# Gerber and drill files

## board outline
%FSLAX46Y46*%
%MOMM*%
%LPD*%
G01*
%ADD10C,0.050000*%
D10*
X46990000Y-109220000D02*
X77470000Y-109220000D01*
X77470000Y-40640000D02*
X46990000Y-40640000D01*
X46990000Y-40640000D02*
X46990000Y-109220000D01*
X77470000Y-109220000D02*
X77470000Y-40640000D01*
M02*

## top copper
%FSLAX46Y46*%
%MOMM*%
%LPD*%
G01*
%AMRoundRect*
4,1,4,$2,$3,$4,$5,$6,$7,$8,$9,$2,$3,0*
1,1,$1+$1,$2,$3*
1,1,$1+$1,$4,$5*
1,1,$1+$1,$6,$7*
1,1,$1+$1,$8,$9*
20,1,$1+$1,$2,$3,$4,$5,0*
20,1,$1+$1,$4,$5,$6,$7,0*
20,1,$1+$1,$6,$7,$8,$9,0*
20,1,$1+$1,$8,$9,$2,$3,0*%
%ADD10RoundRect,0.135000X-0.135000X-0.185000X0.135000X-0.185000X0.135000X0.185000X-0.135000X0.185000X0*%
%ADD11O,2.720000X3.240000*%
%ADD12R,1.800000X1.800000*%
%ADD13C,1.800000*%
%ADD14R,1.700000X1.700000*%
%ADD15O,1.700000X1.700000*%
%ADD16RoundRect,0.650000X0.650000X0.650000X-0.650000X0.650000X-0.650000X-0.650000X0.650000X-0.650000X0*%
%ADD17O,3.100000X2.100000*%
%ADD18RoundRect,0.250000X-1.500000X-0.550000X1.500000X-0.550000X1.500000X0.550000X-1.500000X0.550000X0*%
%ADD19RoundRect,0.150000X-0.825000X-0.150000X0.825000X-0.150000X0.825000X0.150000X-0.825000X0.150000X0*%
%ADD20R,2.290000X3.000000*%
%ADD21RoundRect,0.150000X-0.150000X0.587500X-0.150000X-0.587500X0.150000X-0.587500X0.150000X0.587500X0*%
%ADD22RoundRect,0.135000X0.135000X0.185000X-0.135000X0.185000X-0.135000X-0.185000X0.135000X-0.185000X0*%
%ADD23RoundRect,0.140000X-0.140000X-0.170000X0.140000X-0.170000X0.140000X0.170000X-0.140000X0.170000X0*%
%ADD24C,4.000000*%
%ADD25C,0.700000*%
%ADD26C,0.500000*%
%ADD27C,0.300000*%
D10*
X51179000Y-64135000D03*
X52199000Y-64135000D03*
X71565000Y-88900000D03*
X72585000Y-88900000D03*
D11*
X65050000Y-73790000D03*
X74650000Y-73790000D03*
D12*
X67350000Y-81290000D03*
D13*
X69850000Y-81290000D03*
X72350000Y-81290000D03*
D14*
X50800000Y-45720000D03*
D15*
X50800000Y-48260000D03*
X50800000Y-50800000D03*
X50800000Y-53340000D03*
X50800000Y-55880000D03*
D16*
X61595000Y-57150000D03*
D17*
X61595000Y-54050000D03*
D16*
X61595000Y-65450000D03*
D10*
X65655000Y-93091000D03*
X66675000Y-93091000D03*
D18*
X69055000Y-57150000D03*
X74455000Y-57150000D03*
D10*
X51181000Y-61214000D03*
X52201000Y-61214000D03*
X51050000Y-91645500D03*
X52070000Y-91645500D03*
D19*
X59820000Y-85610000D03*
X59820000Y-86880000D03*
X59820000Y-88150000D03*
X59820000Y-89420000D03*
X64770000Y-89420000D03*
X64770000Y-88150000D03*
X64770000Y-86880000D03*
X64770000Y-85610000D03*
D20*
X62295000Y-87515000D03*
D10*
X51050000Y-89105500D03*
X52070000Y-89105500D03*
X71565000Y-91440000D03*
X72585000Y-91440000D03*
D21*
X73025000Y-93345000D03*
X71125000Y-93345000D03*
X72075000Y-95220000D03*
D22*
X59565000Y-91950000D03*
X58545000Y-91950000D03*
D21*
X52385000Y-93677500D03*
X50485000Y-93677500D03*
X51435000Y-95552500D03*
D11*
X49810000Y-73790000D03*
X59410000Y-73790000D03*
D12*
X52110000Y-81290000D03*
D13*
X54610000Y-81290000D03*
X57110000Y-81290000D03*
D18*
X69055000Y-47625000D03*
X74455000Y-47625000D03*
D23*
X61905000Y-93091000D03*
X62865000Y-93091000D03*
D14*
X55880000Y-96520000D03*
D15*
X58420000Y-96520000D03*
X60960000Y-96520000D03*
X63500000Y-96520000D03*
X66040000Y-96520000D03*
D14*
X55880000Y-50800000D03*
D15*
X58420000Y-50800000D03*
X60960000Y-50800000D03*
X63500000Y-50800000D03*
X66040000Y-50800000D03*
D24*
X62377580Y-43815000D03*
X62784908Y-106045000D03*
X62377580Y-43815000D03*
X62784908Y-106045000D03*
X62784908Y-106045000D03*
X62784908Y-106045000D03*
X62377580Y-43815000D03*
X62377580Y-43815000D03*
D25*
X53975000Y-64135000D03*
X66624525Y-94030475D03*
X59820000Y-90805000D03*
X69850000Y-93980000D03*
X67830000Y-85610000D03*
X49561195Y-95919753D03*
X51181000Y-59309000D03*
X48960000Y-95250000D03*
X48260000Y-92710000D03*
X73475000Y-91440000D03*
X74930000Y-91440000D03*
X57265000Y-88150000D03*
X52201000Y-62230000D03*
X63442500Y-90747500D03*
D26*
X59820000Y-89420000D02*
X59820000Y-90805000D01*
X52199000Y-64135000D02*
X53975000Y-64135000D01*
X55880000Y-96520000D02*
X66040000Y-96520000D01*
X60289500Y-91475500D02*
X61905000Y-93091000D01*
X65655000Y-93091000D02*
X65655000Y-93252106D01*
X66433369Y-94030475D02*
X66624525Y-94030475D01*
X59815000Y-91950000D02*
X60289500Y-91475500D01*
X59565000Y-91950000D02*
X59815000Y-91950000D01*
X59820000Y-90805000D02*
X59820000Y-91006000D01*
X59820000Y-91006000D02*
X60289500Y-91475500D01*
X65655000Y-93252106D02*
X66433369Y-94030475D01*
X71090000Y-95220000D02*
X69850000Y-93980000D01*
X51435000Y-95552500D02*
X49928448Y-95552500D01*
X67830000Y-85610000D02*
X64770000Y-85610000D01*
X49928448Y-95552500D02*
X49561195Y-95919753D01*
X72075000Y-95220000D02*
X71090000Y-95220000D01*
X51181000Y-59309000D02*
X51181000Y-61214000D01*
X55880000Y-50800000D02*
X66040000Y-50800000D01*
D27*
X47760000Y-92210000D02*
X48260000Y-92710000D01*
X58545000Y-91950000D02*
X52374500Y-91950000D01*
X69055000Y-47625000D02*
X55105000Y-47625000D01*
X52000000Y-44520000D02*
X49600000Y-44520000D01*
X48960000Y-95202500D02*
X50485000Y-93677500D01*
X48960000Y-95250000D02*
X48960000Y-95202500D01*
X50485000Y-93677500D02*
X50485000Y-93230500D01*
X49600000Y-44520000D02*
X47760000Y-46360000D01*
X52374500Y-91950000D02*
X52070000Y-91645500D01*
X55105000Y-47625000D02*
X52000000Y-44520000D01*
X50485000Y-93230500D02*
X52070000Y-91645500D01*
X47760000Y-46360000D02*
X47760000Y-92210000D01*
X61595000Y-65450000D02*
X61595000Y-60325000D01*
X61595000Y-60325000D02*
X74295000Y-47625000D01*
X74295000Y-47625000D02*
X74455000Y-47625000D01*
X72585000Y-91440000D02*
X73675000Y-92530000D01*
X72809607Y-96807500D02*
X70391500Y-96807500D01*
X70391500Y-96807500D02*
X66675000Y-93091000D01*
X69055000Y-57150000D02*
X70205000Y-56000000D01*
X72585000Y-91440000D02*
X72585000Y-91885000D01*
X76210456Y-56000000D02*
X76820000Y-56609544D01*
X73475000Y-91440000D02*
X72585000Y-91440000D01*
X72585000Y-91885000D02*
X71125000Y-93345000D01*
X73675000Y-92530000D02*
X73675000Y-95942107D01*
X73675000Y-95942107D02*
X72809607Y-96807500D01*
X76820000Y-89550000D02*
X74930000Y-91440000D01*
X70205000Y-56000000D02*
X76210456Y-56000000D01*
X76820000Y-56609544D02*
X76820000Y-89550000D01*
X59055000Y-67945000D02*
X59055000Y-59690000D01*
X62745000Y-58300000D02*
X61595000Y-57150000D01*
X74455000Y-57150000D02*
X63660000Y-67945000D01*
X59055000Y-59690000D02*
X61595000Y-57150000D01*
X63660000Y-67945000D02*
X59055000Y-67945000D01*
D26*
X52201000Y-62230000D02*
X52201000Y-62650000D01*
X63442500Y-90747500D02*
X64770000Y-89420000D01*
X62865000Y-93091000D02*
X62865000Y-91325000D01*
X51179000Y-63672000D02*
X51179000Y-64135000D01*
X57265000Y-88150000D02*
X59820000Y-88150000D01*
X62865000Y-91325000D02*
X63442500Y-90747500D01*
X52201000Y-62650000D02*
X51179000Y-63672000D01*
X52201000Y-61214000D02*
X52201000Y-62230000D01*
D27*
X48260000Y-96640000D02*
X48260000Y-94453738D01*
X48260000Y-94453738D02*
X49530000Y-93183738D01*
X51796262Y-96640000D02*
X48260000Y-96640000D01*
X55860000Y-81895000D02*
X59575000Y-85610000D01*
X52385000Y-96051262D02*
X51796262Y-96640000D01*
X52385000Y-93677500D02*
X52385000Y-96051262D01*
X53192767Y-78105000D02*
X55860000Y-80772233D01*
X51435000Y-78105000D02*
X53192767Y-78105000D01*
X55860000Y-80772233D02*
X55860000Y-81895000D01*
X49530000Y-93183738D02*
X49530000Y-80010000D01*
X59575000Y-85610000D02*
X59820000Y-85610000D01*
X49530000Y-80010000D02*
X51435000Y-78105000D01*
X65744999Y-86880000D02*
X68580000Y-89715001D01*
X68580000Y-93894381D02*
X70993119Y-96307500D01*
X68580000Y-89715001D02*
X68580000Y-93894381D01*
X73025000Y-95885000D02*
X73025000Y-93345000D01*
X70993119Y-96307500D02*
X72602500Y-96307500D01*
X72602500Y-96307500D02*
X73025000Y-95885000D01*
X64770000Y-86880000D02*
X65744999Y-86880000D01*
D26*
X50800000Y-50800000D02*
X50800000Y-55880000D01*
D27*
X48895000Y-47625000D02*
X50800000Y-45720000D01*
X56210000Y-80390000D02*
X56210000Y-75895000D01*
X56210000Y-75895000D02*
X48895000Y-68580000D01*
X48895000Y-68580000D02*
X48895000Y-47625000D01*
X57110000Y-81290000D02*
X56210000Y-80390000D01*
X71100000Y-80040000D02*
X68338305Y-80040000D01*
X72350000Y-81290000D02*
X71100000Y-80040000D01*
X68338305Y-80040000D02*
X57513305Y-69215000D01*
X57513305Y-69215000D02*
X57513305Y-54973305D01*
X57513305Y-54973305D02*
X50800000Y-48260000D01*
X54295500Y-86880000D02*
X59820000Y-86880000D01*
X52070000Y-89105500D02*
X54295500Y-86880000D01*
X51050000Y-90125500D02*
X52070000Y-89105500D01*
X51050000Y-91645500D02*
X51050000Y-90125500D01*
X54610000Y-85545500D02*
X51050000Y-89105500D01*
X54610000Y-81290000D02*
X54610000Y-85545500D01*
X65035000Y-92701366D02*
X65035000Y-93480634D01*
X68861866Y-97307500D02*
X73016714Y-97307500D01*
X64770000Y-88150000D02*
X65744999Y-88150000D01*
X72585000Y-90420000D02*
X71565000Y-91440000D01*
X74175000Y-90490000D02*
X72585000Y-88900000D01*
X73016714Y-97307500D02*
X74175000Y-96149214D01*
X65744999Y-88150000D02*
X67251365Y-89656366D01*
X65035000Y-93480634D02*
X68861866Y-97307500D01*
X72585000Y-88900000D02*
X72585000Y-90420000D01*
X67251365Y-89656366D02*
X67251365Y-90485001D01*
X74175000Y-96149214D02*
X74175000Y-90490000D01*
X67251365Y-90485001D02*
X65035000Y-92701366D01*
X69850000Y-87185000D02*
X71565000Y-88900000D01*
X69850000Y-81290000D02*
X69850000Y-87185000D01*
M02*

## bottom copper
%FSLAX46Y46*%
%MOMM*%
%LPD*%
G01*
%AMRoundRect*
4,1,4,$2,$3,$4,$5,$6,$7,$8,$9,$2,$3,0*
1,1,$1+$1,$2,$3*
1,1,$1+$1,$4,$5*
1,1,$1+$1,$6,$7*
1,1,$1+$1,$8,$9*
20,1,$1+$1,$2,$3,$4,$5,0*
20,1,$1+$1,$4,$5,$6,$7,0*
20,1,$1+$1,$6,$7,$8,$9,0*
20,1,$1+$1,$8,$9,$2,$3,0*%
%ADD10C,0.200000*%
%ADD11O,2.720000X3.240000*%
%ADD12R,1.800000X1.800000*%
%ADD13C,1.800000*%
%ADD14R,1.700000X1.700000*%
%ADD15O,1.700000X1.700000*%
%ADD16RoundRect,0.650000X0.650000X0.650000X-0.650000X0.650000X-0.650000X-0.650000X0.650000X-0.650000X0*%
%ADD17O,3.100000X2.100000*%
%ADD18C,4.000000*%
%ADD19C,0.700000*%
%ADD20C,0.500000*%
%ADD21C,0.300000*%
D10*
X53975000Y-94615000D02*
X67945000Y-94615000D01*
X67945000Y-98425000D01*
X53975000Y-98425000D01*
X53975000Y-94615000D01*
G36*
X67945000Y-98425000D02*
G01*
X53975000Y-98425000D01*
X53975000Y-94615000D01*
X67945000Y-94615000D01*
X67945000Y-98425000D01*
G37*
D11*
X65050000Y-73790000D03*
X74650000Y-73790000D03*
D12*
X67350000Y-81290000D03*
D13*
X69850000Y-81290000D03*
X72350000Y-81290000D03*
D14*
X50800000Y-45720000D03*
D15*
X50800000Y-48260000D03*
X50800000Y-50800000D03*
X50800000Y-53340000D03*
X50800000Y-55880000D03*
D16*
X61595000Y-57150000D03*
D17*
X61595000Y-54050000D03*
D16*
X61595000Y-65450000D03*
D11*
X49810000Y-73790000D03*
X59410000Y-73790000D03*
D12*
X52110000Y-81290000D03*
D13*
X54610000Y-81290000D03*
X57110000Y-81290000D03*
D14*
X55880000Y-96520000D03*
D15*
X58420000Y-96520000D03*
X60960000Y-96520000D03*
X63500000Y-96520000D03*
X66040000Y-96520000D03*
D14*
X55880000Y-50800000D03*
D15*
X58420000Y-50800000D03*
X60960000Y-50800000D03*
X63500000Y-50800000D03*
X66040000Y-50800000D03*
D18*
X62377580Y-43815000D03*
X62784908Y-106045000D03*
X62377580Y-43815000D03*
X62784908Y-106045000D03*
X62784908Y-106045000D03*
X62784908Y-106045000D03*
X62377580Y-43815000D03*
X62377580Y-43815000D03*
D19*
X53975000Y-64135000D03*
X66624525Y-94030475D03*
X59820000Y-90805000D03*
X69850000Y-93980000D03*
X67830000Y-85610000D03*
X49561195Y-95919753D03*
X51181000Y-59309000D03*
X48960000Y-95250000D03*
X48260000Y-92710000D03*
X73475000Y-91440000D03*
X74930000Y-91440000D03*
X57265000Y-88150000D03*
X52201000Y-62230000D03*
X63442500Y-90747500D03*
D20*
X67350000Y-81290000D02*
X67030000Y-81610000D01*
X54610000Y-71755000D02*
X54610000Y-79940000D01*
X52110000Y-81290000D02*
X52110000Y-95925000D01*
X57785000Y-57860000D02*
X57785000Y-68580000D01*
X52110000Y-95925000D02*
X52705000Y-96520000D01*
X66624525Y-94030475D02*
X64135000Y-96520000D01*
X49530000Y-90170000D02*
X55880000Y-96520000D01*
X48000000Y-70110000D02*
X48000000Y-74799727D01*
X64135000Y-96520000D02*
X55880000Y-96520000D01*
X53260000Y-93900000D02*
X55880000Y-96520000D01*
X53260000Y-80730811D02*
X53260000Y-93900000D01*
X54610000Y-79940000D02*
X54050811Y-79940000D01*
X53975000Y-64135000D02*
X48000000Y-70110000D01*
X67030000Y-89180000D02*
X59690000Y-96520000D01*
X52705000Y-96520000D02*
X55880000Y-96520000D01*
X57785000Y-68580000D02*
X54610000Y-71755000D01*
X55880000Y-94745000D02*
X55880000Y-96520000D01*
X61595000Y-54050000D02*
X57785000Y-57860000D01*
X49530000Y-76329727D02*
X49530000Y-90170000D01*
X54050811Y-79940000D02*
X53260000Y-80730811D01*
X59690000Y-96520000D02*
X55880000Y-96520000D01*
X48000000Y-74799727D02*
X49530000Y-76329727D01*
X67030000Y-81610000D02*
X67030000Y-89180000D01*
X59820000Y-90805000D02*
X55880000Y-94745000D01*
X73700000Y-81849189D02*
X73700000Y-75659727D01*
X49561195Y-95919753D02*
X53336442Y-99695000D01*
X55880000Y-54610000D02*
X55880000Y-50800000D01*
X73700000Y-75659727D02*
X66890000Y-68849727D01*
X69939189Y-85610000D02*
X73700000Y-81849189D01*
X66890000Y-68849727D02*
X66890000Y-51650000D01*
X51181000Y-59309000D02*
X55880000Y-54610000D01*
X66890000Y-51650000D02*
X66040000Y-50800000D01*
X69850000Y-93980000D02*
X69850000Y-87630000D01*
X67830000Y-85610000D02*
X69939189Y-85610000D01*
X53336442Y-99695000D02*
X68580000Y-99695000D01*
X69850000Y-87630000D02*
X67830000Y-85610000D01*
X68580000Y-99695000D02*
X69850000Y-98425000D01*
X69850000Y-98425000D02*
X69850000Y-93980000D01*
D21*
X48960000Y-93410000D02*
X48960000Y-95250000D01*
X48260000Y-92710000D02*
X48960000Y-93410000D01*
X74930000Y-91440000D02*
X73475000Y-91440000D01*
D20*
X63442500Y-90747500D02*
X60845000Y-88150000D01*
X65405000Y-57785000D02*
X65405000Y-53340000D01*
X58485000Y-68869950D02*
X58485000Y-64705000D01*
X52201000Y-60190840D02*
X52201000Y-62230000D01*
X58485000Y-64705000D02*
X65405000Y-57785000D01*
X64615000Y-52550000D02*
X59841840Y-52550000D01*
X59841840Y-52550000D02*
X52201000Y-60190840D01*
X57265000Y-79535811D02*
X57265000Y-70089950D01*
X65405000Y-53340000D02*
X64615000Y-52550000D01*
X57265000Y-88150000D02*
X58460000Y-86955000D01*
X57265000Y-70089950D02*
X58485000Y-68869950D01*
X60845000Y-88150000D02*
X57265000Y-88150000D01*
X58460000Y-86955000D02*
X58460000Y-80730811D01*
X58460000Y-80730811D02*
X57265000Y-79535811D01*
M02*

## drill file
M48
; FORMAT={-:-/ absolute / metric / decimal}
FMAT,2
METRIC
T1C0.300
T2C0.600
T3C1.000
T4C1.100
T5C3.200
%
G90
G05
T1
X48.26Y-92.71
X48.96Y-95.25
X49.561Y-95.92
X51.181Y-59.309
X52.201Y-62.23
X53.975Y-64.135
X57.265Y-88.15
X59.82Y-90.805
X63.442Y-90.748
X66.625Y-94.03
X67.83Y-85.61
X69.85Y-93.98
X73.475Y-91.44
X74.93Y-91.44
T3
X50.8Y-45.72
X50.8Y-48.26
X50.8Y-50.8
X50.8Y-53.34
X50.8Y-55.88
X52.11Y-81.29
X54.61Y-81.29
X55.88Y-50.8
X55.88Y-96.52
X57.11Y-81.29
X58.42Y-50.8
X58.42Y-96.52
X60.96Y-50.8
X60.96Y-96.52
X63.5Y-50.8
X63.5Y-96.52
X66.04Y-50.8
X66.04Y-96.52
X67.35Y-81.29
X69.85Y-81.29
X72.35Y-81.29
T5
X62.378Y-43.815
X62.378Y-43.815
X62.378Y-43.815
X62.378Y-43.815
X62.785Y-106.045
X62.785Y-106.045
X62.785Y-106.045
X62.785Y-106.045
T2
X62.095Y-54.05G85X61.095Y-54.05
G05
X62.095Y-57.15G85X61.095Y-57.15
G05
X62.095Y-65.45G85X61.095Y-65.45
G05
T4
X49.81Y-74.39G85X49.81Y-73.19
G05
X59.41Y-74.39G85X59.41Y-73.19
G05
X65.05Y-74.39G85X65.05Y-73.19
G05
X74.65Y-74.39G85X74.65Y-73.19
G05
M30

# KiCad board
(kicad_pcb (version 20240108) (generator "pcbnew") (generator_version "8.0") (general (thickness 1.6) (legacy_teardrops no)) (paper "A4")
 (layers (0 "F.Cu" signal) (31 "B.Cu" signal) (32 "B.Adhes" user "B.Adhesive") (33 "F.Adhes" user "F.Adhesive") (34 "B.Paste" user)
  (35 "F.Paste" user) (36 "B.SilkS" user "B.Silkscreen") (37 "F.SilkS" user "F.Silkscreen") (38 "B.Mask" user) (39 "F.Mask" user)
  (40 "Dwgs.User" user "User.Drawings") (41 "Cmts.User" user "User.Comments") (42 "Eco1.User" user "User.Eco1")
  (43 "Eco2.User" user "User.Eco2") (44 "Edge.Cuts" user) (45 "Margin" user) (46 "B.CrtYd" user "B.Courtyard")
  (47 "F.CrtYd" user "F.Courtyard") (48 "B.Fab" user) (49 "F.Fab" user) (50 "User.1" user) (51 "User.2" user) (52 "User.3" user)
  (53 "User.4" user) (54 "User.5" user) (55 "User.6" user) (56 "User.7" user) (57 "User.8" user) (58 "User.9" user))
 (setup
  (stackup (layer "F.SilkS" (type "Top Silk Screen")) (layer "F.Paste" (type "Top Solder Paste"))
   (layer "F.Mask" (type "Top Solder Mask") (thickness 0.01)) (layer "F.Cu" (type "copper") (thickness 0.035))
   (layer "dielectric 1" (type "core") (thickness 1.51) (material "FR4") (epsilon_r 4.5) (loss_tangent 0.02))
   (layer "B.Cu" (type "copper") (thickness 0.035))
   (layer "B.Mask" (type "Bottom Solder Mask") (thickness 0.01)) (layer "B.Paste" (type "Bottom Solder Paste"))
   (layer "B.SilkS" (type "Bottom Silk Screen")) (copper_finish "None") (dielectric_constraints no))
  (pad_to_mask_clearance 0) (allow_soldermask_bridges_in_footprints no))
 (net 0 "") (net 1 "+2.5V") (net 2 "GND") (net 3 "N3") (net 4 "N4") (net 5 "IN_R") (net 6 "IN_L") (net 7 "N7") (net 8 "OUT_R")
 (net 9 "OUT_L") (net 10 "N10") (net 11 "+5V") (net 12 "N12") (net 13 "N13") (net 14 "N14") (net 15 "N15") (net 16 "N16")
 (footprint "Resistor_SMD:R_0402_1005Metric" (layer "F.Cu") (at 51.689 64.135)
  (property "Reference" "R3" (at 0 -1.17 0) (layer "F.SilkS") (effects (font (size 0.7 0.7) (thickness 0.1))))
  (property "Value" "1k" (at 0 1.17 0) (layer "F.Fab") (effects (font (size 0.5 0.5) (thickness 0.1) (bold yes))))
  (pad "1" smd roundrect (at -0.51 0) (size 0.54 0.64) (layers "F.Cu" "F.Paste" "F.Mask") (roundrect_rratio 0.25) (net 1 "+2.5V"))
  (pad "2" smd roundrect (at 0.51 0) (size 0.54 0.64) (layers "F.Cu" "F.Paste" "F.Mask") (roundrect_rratio 0.25) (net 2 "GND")))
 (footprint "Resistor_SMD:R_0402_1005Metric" (layer "F.Cu") (at 72.075 88.9)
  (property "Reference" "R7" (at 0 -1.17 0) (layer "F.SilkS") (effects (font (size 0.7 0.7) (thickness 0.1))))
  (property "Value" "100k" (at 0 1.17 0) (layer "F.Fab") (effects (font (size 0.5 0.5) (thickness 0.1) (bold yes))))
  (pad "1" smd roundrect (at -0.51 0) (size 0.54 0.64) (layers "F.Cu" "F.Paste" "F.Mask") (roundrect_rratio 0.25) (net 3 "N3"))
  (pad "2" smd roundrect (at 0.51 0) (size 0.54 0.64) (layers "F.Cu" "F.Paste" "F.Mask") (roundrect_rratio 0.25) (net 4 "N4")))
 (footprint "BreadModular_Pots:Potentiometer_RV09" (layer "F.Cu") (at 67.35 81.29 90)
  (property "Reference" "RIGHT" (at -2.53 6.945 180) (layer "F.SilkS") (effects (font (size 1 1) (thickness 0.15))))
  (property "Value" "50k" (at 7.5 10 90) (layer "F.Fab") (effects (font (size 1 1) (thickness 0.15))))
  (pad "" thru_hole oval (at 7.5 -2.3 180) (size 2.72 3.24) (drill oval 1.1 2.3) (layers "*.Cu" "*.Mask") (remove_unused_layers no))
  (pad "" thru_hole oval (at 7.5 7.3 180) (size 2.72 3.24) (drill oval 1.1 2.3) (layers "*.Cu" "*.Mask") (remove_unused_layers no))
  (pad "1" thru_hole rect (at 0 0 180) (size 1.8 1.8) (drill 1) (layers "*.Cu" "*.Mask") (remove_unused_layers no) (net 2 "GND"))
  (pad "2" thru_hole circle (at 0 2.5 180) (size 1.8 1.8) (drill 1) (layers "*.Cu" "*.Mask") (remove_unused_layers no) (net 3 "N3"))
  (pad "3" thru_hole circle (at 0 5 180) (size 1.8 1.8) (drill 1) (layers "*.Cu" "*.Mask") (remove_unused_layers no) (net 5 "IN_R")))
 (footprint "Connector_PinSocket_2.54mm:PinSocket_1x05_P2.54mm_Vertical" (layer "F.Cu") (at 50.8 45.72)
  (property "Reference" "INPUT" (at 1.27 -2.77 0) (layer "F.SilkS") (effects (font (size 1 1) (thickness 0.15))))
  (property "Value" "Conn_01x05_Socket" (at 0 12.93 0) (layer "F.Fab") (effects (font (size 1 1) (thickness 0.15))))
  (pad "1" thru_hole rect (at 0 0) (size 1.7 1.7) (drill 1) (layers "*.Cu" "*.Mask") (remove_unused_layers no) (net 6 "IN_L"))
  (pad "2" thru_hole oval (at 0 2.54) (size 1.7 1.7) (drill 1) (layers "*.Cu" "*.Mask") (remove_unused_layers no) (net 5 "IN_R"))
  (pad "3" thru_hole oval (at 0 5.08) (size 1.7 1.7) (drill 1) (layers "*.Cu" "*.Mask") (remove_unused_layers no) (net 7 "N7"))
  (pad "4" thru_hole oval (at 0 7.62) (size 1.7 1.7) (drill 1) (layers "*.Cu" "*.Mask") (remove_unused_layers no) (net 7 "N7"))
  (pad "5" thru_hole oval (at 0 10.16) (size 1.7 1.7) (drill 1) (layers "*.Cu" "*.Mask") (remove_unused_layers no) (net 7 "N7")))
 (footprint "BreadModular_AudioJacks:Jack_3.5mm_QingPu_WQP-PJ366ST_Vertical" (layer "F.Cu") (at 61.595 60.53 180)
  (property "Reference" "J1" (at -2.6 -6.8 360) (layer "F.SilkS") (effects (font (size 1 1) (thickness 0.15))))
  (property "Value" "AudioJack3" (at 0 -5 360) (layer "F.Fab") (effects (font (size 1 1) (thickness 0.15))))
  (pad "R" thru_hole roundrect (at 0 3.38 180) (size 2.6 2.6) (drill oval 1.6 0.6) (layers "*.Cu" "*.Mask") (remove_unused_layers no)
   (roundrect_rratio 0.25) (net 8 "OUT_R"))
  (pad "S" thru_hole oval (at 0 6.48 180) (size 3.1 2.1) (drill oval 1.6 0.6) (layers "*.Cu" "*.Mask") (remove_unused_layers no)
   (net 2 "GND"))
  (pad "T" thru_hole roundrect (at 0 -4.92 180) (size 2.6 2.6) (drill oval 1.6 0.6) (layers "*.Cu" "*.Mask") (remove_unused_layers no)
   (roundrect_rratio 0.25) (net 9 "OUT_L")))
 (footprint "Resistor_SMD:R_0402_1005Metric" (layer "F.Cu") (at 66.165 93.091)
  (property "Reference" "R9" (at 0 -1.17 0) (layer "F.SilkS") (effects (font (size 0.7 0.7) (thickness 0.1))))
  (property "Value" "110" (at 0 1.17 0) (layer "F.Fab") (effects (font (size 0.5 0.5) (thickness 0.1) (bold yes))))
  (pad "1" smd roundrect (at -0.51 0) (size 0.54 0.64) (layers "F.Cu" "F.Paste" "F.Mask") (roundrect_rratio 0.25) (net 2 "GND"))
  (pad "2" smd roundrect (at 0.51 0) (size 0.54 0.64) (layers "F.Cu" "F.Paste" "F.Mask") (roundrect_rratio 0.25) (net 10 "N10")))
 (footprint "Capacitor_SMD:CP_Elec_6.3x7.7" (layer "F.Cu") (at 71.755 57.15)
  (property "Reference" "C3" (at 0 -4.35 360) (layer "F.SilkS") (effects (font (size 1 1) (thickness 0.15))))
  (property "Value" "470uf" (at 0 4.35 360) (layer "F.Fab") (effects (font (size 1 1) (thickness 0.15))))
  (pad "1" smd roundrect (at -2.7 0) (size 3.5 1.6) (layers "F.Cu" "F.Paste" "F.Mask") (roundrect_rratio 0.15625) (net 10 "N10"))
  (pad "2" smd roundrect (at 2.7 0) (size 3.5 1.6) (layers "F.Cu" "F.Paste" "F.Mask") (roundrect_rratio 0.15625) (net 8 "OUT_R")))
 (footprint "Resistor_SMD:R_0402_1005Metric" (layer "F.Cu") (at 51.691 61.214)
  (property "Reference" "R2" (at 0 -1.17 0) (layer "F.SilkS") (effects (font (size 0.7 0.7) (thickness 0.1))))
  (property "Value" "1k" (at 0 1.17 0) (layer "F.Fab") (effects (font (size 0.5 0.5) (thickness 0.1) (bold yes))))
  (pad "1" smd roundrect (at -0.51 0) (size 0.54 0.64) (layers "F.Cu" "F.Paste" "F.Mask") (roundrect_rratio 0.25) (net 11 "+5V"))
  (pad "2" smd roundrect (at 0.51 0) (size 0.54 0.64) (layers "F.Cu" "F.Paste" "F.Mask") (roundrect_rratio 0.25) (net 1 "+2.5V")))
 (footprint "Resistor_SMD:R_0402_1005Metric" (layer "F.Cu") (at 51.56 91.6455)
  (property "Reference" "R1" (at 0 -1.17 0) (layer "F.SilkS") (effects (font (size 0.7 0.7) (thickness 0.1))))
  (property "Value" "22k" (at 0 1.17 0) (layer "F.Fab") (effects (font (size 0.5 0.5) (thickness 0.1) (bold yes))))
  (pad "1" smd roundrect (at -0.51 0) (size 0.54 0.64) (layers "F.Cu" "F.Paste" "F.Mask") (roundrect_rratio 0.25) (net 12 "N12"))
  (pad "2" smd roundrect (at 0.51 0) (size 0.54 0.64) (layers "F.Cu" "F.Paste" "F.Mask") (roundrect_rratio 0.25) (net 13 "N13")))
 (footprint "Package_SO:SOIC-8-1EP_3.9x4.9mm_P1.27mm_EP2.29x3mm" (layer "F.Cu") (at 62.295 87.515)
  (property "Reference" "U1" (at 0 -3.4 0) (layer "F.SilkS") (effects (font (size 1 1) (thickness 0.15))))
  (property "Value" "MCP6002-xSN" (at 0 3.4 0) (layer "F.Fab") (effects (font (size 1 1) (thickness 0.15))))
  (pad "" smd roundrect (at -0.57 -0.75) (size 0.92 1.21) (layers "F.Paste") (roundrect_rratio 0.25))
  (pad "" smd roundrect (at -0.57 0.75) (size 0.92 1.21) (layers "F.Paste") (roundrect_rratio 0.25))
  (pad "" smd roundrect (at 0.57 -0.75) (size 0.92 1.21) (layers "F.Paste") (roundrect_rratio 0.25))
  (pad "" smd roundrect (at 0.57 0.75) (size 0.92 1.21) (layers "F.Paste") (roundrect_rratio 0.25))
  (pad "1" smd roundrect (at -2.475 -1.905) (size 1.95 0.6) (layers "F.Cu" "F.Paste" "F.Mask") (roundrect_rratio 0.25) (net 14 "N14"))
  (pad "2" smd roundrect (at -2.475 -0.635) (size 1.95 0.6) (layers "F.Cu" "F.Paste" "F.Mask") (roundrect_rratio 0.25) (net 12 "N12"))
  (pad "3" smd roundrect (at -2.475 0.635) (size 1.95 0.6) (layers "F.Cu" "F.Paste" "F.Mask") (roundrect_rratio 0.25) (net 1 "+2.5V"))
  (pad "4" smd roundrect (at -2.475 1.905) (size 1.95 0.6) (layers "F.Cu" "F.Paste" "F.Mask") (roundrect_rratio 0.25) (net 2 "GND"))
  (pad "5" smd roundrect (at 2.475 1.905) (size 1.95 0.6) (layers "F.Cu" "F.Paste" "F.Mask") (roundrect_rratio 0.25) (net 1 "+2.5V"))
  (pad "6" smd roundrect (at 2.475 0.635) (size 1.95 0.6) (layers "F.Cu" "F.Paste" "F.Mask") (roundrect_rratio 0.25) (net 4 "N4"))
  (pad "7" smd roundrect (at 2.475 -0.635) (size 1.95 0.6) (layers "F.Cu" "F.Paste" "F.Mask") (roundrect_rratio 0.25) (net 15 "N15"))
  (pad "8" smd roundrect (at 2.475 -1.905) (size 1.95 0.6) (layers "F.Cu" "F.Paste" "F.Mask") (roundrect_rratio 0.25) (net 11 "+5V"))
  (pad "9" smd rect (at 0 0) (size 2.29 3) (layers "F.Cu" "F.Mask") (zone_connect 2)))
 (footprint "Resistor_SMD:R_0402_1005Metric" (layer "F.Cu") (at 51.56 89.1055)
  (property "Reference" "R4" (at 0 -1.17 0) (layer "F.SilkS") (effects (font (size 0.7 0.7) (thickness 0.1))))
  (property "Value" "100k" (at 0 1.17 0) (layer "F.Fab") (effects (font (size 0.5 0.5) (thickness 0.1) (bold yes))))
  (pad "1" smd roundrect (at -0.51 0) (size 0.54 0.64) (layers "F.Cu" "F.Paste" "F.Mask") (roundrect_rratio 0.25) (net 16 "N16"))
  (pad "2" smd roundrect (at 0.51 0) (size 0.54 0.64) (layers "F.Cu" "F.Paste" "F.Mask") (roundrect_rratio 0.25) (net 12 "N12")))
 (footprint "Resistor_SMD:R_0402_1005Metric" (layer "F.Cu") (at 72.075 91.44)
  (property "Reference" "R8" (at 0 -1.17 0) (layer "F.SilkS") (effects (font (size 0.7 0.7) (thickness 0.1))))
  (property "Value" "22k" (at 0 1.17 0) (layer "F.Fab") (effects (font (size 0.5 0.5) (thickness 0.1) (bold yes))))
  (pad "1" smd roundrect (at -0.51 0) (size 0.54 0.64) (layers "F.Cu" "F.Paste" "F.Mask") (roundrect_rratio 0.25) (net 4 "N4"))
  (pad "2" smd roundrect (at 0.51 0) (size 0.54 0.64) (layers "F.Cu" "F.Paste" "F.Mask") (roundrect_rratio 0.25) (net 10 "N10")))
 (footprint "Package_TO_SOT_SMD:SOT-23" (layer "F.Cu") (at 72.075 94.2825 -90)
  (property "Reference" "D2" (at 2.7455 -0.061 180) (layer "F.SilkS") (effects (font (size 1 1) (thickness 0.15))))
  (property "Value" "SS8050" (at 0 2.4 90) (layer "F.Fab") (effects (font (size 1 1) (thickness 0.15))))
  (pad "1" smd roundrect (at -0.9375 -0.95 270) (size 1.475 0.6) (layers "F.Cu" "F.Paste" "F.Mask") (roundrect_rratio 0.25) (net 15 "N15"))
  (pad "2" smd roundrect (at -0.9375 0.95 270) (size 1.475 0.6) (layers "F.Cu" "F.Paste" "F.Mask") (roundrect_rratio 0.25) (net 10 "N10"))
  (pad "3" smd roundrect (at 0.9375 0 270) (size 1.475 0.6) (layers "F.Cu" "F.Paste" "F.Mask") (roundrect_rratio 0.25) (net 11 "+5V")))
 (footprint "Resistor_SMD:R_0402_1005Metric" (layer "F.Cu") (at 59.055 91.95 180)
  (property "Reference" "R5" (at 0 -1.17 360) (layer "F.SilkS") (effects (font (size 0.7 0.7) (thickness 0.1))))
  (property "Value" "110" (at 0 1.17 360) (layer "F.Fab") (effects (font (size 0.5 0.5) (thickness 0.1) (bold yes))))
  (pad "1" smd roundrect (at -0.51 0 180) (size 0.54 0.64) (layers "F.Cu" "F.Paste" "F.Mask") (roundrect_rratio 0.25) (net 2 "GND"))
  (pad "2" smd roundrect (at 0.51 0 180) (size 0.54 0.64) (layers "F.Cu" "F.Paste" "F.Mask") (roundrect_rratio 0.25) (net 13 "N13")))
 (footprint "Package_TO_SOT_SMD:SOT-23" (layer "F.Cu") (at 51.435 94.615 -90)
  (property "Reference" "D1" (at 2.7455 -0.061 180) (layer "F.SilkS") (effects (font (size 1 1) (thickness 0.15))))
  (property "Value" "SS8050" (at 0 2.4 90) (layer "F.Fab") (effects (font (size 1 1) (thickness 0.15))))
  (pad "1" smd roundrect (at -0.9375 -0.95 270) (size 1.475 0.6) (layers "F.Cu" "F.Paste" "F.Mask") (roundrect_rratio 0.25) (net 14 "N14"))
  (pad "2" smd roundrect (at -0.9375 0.95 270) (size 1.475 0.6) (layers "F.Cu" "F.Paste" "F.Mask") (roundrect_rratio 0.25) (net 13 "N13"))
  (pad "3" smd roundrect (at 0.9375 0 270) (size 1.475 0.6) (layers "F.Cu" "F.Paste" "F.Mask") (roundrect_rratio 0.25) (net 11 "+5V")))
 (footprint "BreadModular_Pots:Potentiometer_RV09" (layer "F.Cu") (at 52.11 81.29 90)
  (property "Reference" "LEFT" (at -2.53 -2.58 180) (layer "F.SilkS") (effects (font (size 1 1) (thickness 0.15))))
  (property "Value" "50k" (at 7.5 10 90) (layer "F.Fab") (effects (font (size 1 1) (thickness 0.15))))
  (pad "" thru_hole oval (at 7.5 -2.3 180) (size 2.72 3.24) (drill oval 1.1 2.3) (layers "*.Cu" "*.Mask") (remove_unused_layers no))
  (pad "" thru_hole oval (at 7.5 7.3 180) (size 2.72 3.24) (drill oval 1.1 2.3) (layers "*.Cu" "*.Mask") (remove_unused_layers no))
  (pad "1" thru_hole rect (at 0 0 180) (size 1.8 1.8) (drill 1) (layers "*.Cu" "*.Mask") (remove_unused_layers no) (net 2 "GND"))
  (pad "2" thru_hole circle (at 0 2.5 180) (size 1.8 1.8) (drill 1) (layers "*.Cu" "*.Mask") (remove_unused_layers no) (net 16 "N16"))
  (pad "3" thru_hole circle (at 0 5 180) (size 1.8 1.8) (drill 1) (layers "*.Cu" "*.Mask") (remove_unused_layers no) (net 6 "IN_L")))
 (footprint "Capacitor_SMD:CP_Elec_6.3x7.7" (layer "F.Cu") (at 71.755 47.625)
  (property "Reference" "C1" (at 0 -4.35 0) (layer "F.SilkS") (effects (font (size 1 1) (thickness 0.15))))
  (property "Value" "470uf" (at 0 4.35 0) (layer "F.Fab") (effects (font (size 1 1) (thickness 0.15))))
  (pad "1" smd roundrect (at -2.7 0) (size 3.5 1.6) (layers "F.Cu" "F.Paste" "F.Mask") (roundrect_rratio 0.15625) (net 13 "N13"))
  (pad "2" smd roundrect (at 2.7 0) (size 3.5 1.6) (layers "F.Cu" "F.Paste" "F.Mask") (roundrect_rratio 0.15625) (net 9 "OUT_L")))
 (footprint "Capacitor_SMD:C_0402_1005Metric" (layer "F.Cu") (at 62.385 93.091)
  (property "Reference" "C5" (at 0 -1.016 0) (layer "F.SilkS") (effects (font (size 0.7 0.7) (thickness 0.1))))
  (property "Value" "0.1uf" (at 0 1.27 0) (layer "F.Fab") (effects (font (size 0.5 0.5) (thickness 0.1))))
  (pad "1" smd roundrect (at -0.48 0) (size 0.56 0.62) (layers "F.Cu" "F.Paste" "F.Mask") (roundrect_rratio 0.25) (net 2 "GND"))
  (pad "2" smd roundrect (at 0.48 0) (size 0.56 0.62) (layers "F.Cu" "F.Paste" "F.Mask") (roundrect_rratio 0.25) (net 1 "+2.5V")))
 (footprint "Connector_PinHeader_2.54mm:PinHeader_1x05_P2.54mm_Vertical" (layer "B.Cu") (at 55.88 96.52 -90)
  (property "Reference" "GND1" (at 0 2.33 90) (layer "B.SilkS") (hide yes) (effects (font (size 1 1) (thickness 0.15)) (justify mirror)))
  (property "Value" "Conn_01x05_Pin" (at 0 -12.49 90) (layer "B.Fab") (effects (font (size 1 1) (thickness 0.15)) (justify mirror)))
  (pad "1" thru_hole rect (at 0 0 270) (size 1.7 1.7) (drill 1) (layers "*.Cu" "*.Mask") (remove_unused_layers no) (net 2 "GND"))
  (pad "2" thru_hole oval (at 0 -2.54 270) (size 1.7 1.7) (drill 1) (layers "*.Cu" "*.Mask") (remove_unused_layers no) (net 2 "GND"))
  (pad "3" thru_hole oval (at 0 -5.08 270) (size 1.7 1.7) (drill 1) (layers "*.Cu" "*.Mask") (remove_unused_layers no) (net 2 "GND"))
  (pad "4" thru_hole oval (at 0 -7.62 270) (size 1.7 1.7) (drill 1) (layers "*.Cu" "*.Mask") (remove_unused_layers no) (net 2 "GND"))
  (pad "5" thru_hole oval (at 0 -10.16 270) (size 1.7 1.7) (drill 1) (layers "*.Cu" "*.Mask") (remove_unused_layers no) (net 2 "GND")))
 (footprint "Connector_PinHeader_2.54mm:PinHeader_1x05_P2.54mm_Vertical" (layer "B.Cu") (at 55.88 50.8 -90)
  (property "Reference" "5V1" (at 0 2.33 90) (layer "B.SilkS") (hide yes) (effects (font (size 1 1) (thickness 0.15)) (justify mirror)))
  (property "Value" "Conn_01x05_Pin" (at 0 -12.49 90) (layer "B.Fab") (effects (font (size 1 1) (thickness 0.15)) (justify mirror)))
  (pad "1" thru_hole rect (at 0 0 270) (size 1.7 1.7) (drill 1) (layers "*.Cu" "*.Mask") (remove_unused_layers no) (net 11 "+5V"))
  (pad "2" thru_hole oval (at 0 -2.54 270) (size 1.7 1.7) (drill 1) (layers "*.Cu" "*.Mask") (remove_unused_layers no) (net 11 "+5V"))
  (pad "3" thru_hole oval (at 0 -5.08 270) (size 1.7 1.7) (drill 1) (layers "*.Cu" "*.Mask") (remove_unused_layers no) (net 11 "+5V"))
  (pad "4" thru_hole oval (at 0 -7.62 270) (size 1.7 1.7) (drill 1) (layers "*.Cu" "*.Mask") (remove_unused_layers no) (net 11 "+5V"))
  (pad "5" thru_hole oval (at 0 -10.16 270) (size 1.7 1.7) (drill 1) (layers "*.Cu" "*.Mask") (remove_unused_layers no) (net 11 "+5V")))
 (gr_poly
  (pts (xy 53.975 94.615) (xy 67.945 94.615) (xy 67.945 98.425) (xy 53.975 98.425)) (stroke (width 0.2) (type solid)) (fill solid)
  (layer "B.Cu") (net 2))
 (gr_line (start 46.99 109.22) (end 77.47 109.22) (stroke (width 0.05) (type default)) (layer "Edge.Cuts"))
 (gr_line (start 77.47 40.64) (end 46.99 40.64) (stroke (width 0.05) (type default)) (layer "Edge.Cuts"))
 (gr_line (start 46.99 40.64) (end 46.99 109.22) (stroke (width 0.05) (type default)) (layer "Edge.Cuts"))
 (gr_line (start 77.47 109.22) (end 77.47 40.64) (stroke (width 0.05) (type default)) (layer "Edge.Cuts"))
 (via (at 62.37758 43.815) (size 4) (drill 3.2) (layers "F.Cu" "B.Cu") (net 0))
 (via (at 62.784908 106.045) (size 4) (drill 3.2) (layers "F.Cu" "B.Cu") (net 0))
 (via (at 62.37758 43.815) (size 4) (drill 3.2) (layers "F.Cu" "B.Cu") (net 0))
 (via (at 62.784908 106.045) (size 4) (drill 3.2) (layers "F.Cu" "B.Cu") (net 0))
 (via (at 62.784908 106.045) (size 4) (drill 3.2) (layers "F.Cu" "B.Cu") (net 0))
 (via (at 62.784908 106.045) (size 4) (drill 3.2) (layers "F.Cu" "B.Cu") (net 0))
 (via (at 62.37758 43.815) (size 4) (drill 3.2) (layers "F.Cu" "B.Cu") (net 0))
 (via (at 62.37758 43.815) (size 4) (drill 3.2) (layers "F.Cu" "B.Cu") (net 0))
 (segment (start 59.82 89.42) (end 59.82 90.805) (width 0.5) (layer "F.Cu") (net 2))
 (segment (start 52.199 64.135) (end 53.975 64.135) (width 0.5) (layer "F.Cu") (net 2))
 (segment (start 55.88 96.52) (end 66.04 96.52) (width 0.5) (layer "F.Cu") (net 2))
 (segment (start 60.2895 91.4755) (end 61.905 93.091) (width 0.5) (layer "F.Cu") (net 2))
 (segment (start 65.655 93.091) (end 65.655 93.252106) (width 0.5) (layer "F.Cu") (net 2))
 (segment (start 66.433369 94.030475) (end 66.624525 94.030475) (width 0.5) (layer "F.Cu") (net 2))
 (segment (start 59.815 91.95) (end 60.2895 91.4755) (width 0.5) (layer "F.Cu") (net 2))
 (segment (start 59.565 91.95) (end 59.815 91.95) (width 0.5) (layer "F.Cu") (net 2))
 (segment (start 59.82 90.805) (end 59.82 91.006) (width 0.5) (layer "F.Cu") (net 2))
 (segment (start 59.82 91.006) (end 60.2895 91.4755) (width 0.5) (layer "F.Cu") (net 2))
 (segment (start 65.655 93.252106) (end 66.433369 94.030475) (width 0.5) (layer "F.Cu") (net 2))
 (via (at 53.975 64.135) (size 0.7) (drill 0.3) (layers "F.Cu" "B.Cu") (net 2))
 (via (at 66.624525 94.030475) (size 0.7) (drill 0.3) (layers "F.Cu" "B.Cu") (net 2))
 (via (at 59.82 90.805) (size 0.7) (drill 0.3) (layers "F.Cu" "B.Cu") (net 2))
 (segment (start 67.35 81.29) (end 67.03 81.61) (width 0.5) (layer "B.Cu") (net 2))
 (segment (start 54.61 71.755) (end 54.61 79.94) (width 0.5) (layer "B.Cu") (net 2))
 (segment (start 52.11 81.29) (end 52.11 95.925) (width 0.5) (layer "B.Cu") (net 2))
 (segment (start 57.785 57.86) (end 57.785 68.58) (width 0.5) (layer "B.Cu") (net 2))
 (segment (start 52.11 95.925) (end 52.705 96.52) (width 0.5) (layer "B.Cu") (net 2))
 (segment (start 66.624525 94.030475) (end 64.135 96.52) (width 0.5) (layer "B.Cu") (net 2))
 (segment (start 49.53 90.17) (end 55.88 96.52) (width 0.5) (layer "B.Cu") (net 2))
 (segment (start 48 70.11) (end 48 74.799727) (width 0.5) (layer "B.Cu") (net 2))
 (segment (start 64.135 96.52) (end 55.88 96.52) (width 0.5) (layer "B.Cu") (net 2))
 (segment (start 53.26 93.9) (end 55.88 96.52) (width 0.5) (layer "B.Cu") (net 2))
 (segment (start 53.26 80.730811) (end 53.26 93.9) (width 0.5) (layer "B.Cu") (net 2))
 (segment (start 54.61 79.94) (end 54.050811 79.94) (width 0.5) (layer "B.Cu") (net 2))
 (segment (start 53.975 64.135) (end 48 70.11) (width 0.5) (layer "B.Cu") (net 2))
 (segment (start 67.03 89.18) (end 59.69 96.52) (width 0.5) (layer "B.Cu") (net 2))
 (segment (start 52.705 96.52) (end 55.88 96.52) (width 0.5) (layer "B.Cu") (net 2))
 (segment (start 57.785 68.58) (end 54.61 71.755) (width 0.5) (layer "B.Cu") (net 2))
 (segment (start 55.88 94.745) (end 55.88 96.52) (width 0.5) (layer "B.Cu") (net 2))
 (segment (start 61.595 54.05) (end 57.785 57.86) (width 0.5) (layer "B.Cu") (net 2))
 (segment (start 49.53 76.329727) (end 49.53 90.17) (width 0.5) (layer "B.Cu") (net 2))
 (segment (start 54.050811 79.94) (end 53.26 80.730811) (width 0.5) (layer "B.Cu") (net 2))
 (segment (start 59.69 96.52) (end 55.88 96.52) (width 0.5) (layer "B.Cu") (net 2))
 (segment (start 48 74.799727) (end 49.53 76.329727) (width 0.5) (layer "B.Cu") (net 2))
 (segment (start 67.03 81.61) (end 67.03 89.18) (width 0.5) (layer "B.Cu") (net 2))
 (segment (start 59.82 90.805) (end 55.88 94.745) (width 0.5) (layer "B.Cu") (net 2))
 (segment (start 71.09 95.22) (end 69.85 93.98) (width 0.5) (layer "F.Cu") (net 11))
 (segment (start 51.435 95.5525) (end 49.928448 95.5525) (width 0.5) (layer "F.Cu") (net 11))
 (segment (start 67.83 85.61) (end 64.77 85.61) (width 0.5) (layer "F.Cu") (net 11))
 (segment (start 49.928448 95.5525) (end 49.561195 95.919753) (width 0.5) (layer "F.Cu") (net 11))
 (segment (start 72.075 95.22) (end 71.09 95.22) (width 0.5) (layer "F.Cu") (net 11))
 (segment (start 51.181 59.309) (end 51.181 61.214) (width 0.5) (layer "F.Cu") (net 11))
 (segment (start 55.88 50.8) (end 66.04 50.8) (width 0.5) (layer "F.Cu") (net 11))
 (via (at 69.85 93.98) (size 0.7) (drill 0.3) (layers "F.Cu" "B.Cu") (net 11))
 (via (at 67.83 85.61) (size 0.7) (drill 0.3) (layers "F.Cu" "B.Cu") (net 11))
 (via (at 49.561195 95.919753) (size 0.7) (drill 0.3) (layers "F.Cu" "B.Cu") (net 11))
 (via (at 51.181 59.309) (size 0.7) (drill 0.3) (layers "F.Cu" "B.Cu") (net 11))
 (segment (start 73.7 81.849189) (end 73.7 75.659727) (width 0.5) (layer "B.Cu") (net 11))
 (segment (start 49.561195 95.919753) (end 53.336442 99.695) (width 0.5) (layer "B.Cu") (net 11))
 (segment (start 55.88 54.61) (end 55.88 50.8) (width 0.5) (layer "B.Cu") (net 11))
 (segment (start 73.7 75.659727) (end 66.89 68.849727) (width 0.5) (layer "B.Cu") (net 11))
 (segment (start 69.939189 85.61) (end 73.7 81.849189) (width 0.5) (layer "B.Cu") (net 11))
 (segment (start 66.89 68.849727) (end 66.89 51.65) (width 0.5) (layer "B.Cu") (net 11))
 (segment (start 51.181 59.309) (end 55.88 54.61) (width 0.5) (layer "B.Cu") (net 11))
 (segment (start 66.89 51.65) (end 66.04 50.8) (width 0.5) (layer "B.Cu") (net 11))
 (segment (start 69.85 93.98) (end 69.85 87.63) (width 0.5) (layer "B.Cu") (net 11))
 (segment (start 67.83 85.61) (end 69.939189 85.61) (width 0.5) (layer "B.Cu") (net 11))
 (segment (start 53.336442 99.695) (end 68.58 99.695) (width 0.5) (layer "B.Cu") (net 11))
 (segment (start 69.85 87.63) (end 67.83 85.61) (width 0.5) (layer "B.Cu") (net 11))
 (segment (start 68.58 99.695) (end 69.85 98.425) (width 0.5) (layer "B.Cu") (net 11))
 (segment (start 69.85 98.425) (end 69.85 93.98) (width 0.5) (layer "B.Cu") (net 11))
 (segment (start 47.76 92.21) (end 48.26 92.71) (width 0.3) (layer "F.Cu") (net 13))
 (segment (start 58.545 91.95) (end 52.3745 91.95) (width 0.3) (layer "F.Cu") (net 13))
 (segment (start 69.055 47.625) (end 55.105 47.625) (width 0.3) (layer "F.Cu") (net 13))
 (segment (start 52 44.52) (end 49.6 44.52) (width 0.3) (layer "F.Cu") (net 13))
 (segment (start 48.96 95.2025) (end 50.485 93.6775) (width 0.3) (layer "F.Cu") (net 13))
 (segment (start 48.96 95.25) (end 48.96 95.2025) (width 0.3) (layer "F.Cu") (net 13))
 (segment (start 50.485 93.6775) (end 50.485 93.2305) (width 0.3) (layer "F.Cu") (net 13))
 (segment (start 49.6 44.52) (end 47.76 46.36) (width 0.3) (layer "F.Cu") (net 13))
 (segment (start 52.3745 91.95) (end 52.07 91.6455) (width 0.3) (layer "F.Cu") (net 13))
 (segment (start 55.105 47.625) (end 52 44.52) (width 0.3) (layer "F.Cu") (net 13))
 (segment (start 50.485 93.2305) (end 52.07 91.6455) (width 0.3) (layer "F.Cu") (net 13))
 (segment (start 47.76 46.36) (end 47.76 92.21) (width 0.3) (layer "F.Cu") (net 13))
 (via (at 48.96 95.25) (size 0.7) (drill 0.3) (layers "F.Cu" "B.Cu") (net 13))
 (via (at 48.26 92.71) (size 0.7) (drill 0.3) (layers "F.Cu" "B.Cu") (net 13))
 (segment (start 48.96 93.41) (end 48.96 95.25) (width 0.3) (layer "B.Cu") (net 13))
 (segment (start 48.26 92.71) (end 48.96 93.41) (width 0.3) (layer "B.Cu") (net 13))
 (segment (start 61.595 65.45) (end 61.595 60.325) (width 0.3) (layer "F.Cu") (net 9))
 (segment (start 61.595 60.325) (end 74.295 47.625) (width 0.3) (layer "F.Cu") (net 9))
 (segment (start 74.295 47.625) (end 74.455 47.625) (width 0.3) (layer "F.Cu") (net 9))
 (segment (start 72.585 91.44) (end 73.675 92.53) (width 0.3) (layer "F.Cu") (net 10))
 (segment (start 72.809607 96.8075) (end 70.3915 96.8075) (width 0.3) (layer "F.Cu") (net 10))
 (segment (start 70.3915 96.8075) (end 66.675 93.091) (width 0.3) (layer "F.Cu") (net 10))
 (segment (start 69.055 57.15) (end 70.205 56) (width 0.3) (layer "F.Cu") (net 10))
 (segment (start 72.585 91.44) (end 72.585 91.885) (width 0.3) (layer "F.Cu") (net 10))
 (segment (start 76.210456 56) (end 76.82 56.609544) (width 0.3) (layer "F.Cu") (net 10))
 (segment (start 73.475 91.44) (end 72.585 91.44) (width 0.3) (layer "F.Cu") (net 10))
 (segment (start 72.585 91.885) (end 71.125 93.345) (width 0.3) (layer "F.Cu") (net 10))
 (segment (start 73.675 92.53) (end 73.675 95.942107) (width 0.3) (layer "F.Cu") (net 10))
 (segment (start 73.675 95.942107) (end 72.809607 96.8075) (width 0.3) (layer "F.Cu") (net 10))
 (segment (start 76.82 89.55) (end 74.93 91.44) (width 0.3) (layer "F.Cu") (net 10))
 (segment (start 70.205 56) (end 76.210456 56) (width 0.3) (layer "F.Cu") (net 10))
 (segment (start 76.82 56.609544) (end 76.82 89.55) (width 0.3) (layer "F.Cu") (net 10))
 (via (at 73.475 91.44) (size 0.7) (drill 0.3) (layers "F.Cu" "B.Cu") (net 10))
 (via (at 74.93 91.44) (size 0.7) (drill 0.3) (layers "F.Cu" "B.Cu") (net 10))
 (segment (start 74.93 91.44) (end 73.475 91.44) (width 0.3) (layer "B.Cu") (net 10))
 (segment (start 59.055 67.945) (end 59.055 59.69) (width 0.3) (layer "F.Cu") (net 8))
 (segment (start 62.745 58.3) (end 61.595 57.15) (width 0.3) (layer "F.Cu") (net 8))
 (segment (start 74.455 57.15) (end 63.66 67.945) (width 0.3) (layer "F.Cu") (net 8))
 (segment (start 59.055 59.69) (end 61.595 57.15) (width 0.3) (layer "F.Cu") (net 8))
 (segment (start 63.66 67.945) (end 59.055 67.945) (width 0.3) (layer "F.Cu") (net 8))
 (segment (start 52.201 62.23) (end 52.201 62.65) (width 0.5) (layer "F.Cu") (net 1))
 (segment (start 63.4425 90.7475) (end 64.77 89.42) (width 0.5) (layer "F.Cu") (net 1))
 (segment (start 62.865 93.091) (end 62.865 91.325) (width 0.5) (layer "F.Cu") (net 1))
 (segment (start 51.179 63.672) (end 51.179 64.135) (width 0.5) (layer "F.Cu") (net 1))
 (segment (start 57.265 88.15) (end 59.82 88.15) (width 0.5) (layer "F.Cu") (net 1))
 (segment (start 62.865 91.325) (end 63.4425 90.7475) (width 0.5) (layer "F.Cu") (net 1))
 (segment (start 52.201 62.65) (end 51.179 63.672) (width 0.5) (layer "F.Cu") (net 1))
 (segment (start 52.201 61.214) (end 52.201 62.23) (width 0.5) (layer "F.Cu") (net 1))
 (via (at 57.265 88.15) (size 0.7) (drill 0.3) (layers "F.Cu" "B.Cu") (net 1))
 (via (at 52.201 62.23) (size 0.7) (drill 0.3) (layers "F.Cu" "B.Cu") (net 1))
 (via (at 63.4425 90.7475) (size 0.7) (drill 0.3) (layers "F.Cu" "B.Cu") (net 1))
 (segment (start 63.4425 90.7475) (end 60.845 88.15) (width 0.5) (layer "B.Cu") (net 1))
 (segment (start 65.405 57.785) (end 65.405 53.34) (width 0.5) (layer "B.Cu") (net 1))
 (segment (start 58.485 68.86995) (end 58.485 64.705) (width 0.5) (layer "B.Cu") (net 1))
 (segment (start 52.201 60.19084) (end 52.201 62.23) (width 0.5) (layer "B.Cu") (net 1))
 (segment (start 58.485 64.705) (end 65.405 57.785) (width 0.5) (layer "B.Cu") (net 1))
 (segment (start 64.615 52.55) (end 59.84184 52.55) (width 0.5) (layer "B.Cu") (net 1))
 (segment (start 59.84184 52.55) (end 52.201 60.19084) (width 0.5) (layer "B.Cu") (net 1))
 (segment (start 57.265 79.535811) (end 57.265 70.08995) (width 0.5) (layer "B.Cu") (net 1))
 (segment (start 65.405 53.34) (end 64.615 52.55) (width 0.5) (layer "B.Cu") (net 1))
 (segment (start 57.265 88.15) (end 58.46 86.955) (width 0.5) (layer "B.Cu") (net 1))
 (segment (start 57.265 70.08995) (end 58.485 68.86995) (width 0.5) (layer "B.Cu") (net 1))
 (segment (start 60.845 88.15) (end 57.265 88.15) (width 0.5) (layer "B.Cu") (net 1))
 (segment (start 58.46 86.955) (end 58.46 80.730811) (width 0.5) (layer "B.Cu") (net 1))
 (segment (start 58.46 80.730811) (end 57.265 79.535811) (width 0.5) (layer "B.Cu") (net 1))
 (segment (start 48.26 96.64) (end 48.26 94.453738) (width 0.3) (layer "F.Cu") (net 14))
 (segment (start 48.26 94.453738) (end 49.53 93.183738) (width 0.3) (layer "F.Cu") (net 14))
 (segment (start 51.796262 96.64) (end 48.26 96.64) (width 0.3) (layer "F.Cu") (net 14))
 (segment (start 55.86 81.895) (end 59.575 85.61) (width 0.3) (layer "F.Cu") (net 14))
 (segment (start 52.385 96.051262) (end 51.796262 96.64) (width 0.3) (layer "F.Cu") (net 14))
 (segment (start 52.385 93.6775) (end 52.385 96.051262) (width 0.3) (layer "F.Cu") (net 14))
 (segment (start 53.192767 78.105) (end 55.86 80.772233) (width 0.3) (layer "F.Cu") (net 14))
 (segment (start 51.435 78.105) (end 53.192767 78.105) (width 0.3) (layer "F.Cu") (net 14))
 (segment (start 55.86 80.772233) (end 55.86 81.895) (width 0.3) (layer "F.Cu") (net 14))
 (segment (start 49.53 93.183738) (end 49.53 80.01) (width 0.3) (layer "F.Cu") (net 14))
 (segment (start 59.575 85.61) (end 59.82 85.61) (width 0.3) (layer "F.Cu") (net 14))
 (segment (start 49.53 80.01) (end 51.435 78.105) (width 0.3) (layer "F.Cu") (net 14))
 (segment (start 65.744999 86.88) (end 68.58 89.715001) (width 0.3) (layer "F.Cu") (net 15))
 (segment (start 68.58 93.894381) (end 70.993119 96.3075) (width 0.3) (layer "F.Cu") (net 15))
 (segment (start 68.58 89.715001) (end 68.58 93.894381) (width 0.3) (layer "F.Cu") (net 15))
 (segment (start 73.025 95.885) (end 73.025 93.345) (width 0.3) (layer "F.Cu") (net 15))
 (segment (start 70.993119 96.3075) (end 72.6025 96.3075) (width 0.3) (layer "F.Cu") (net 15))
 (segment (start 72.6025 96.3075) (end 73.025 95.885) (width 0.3) (layer "F.Cu") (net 15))
 (segment (start 64.77 86.88) (end 65.744999 86.88) (width 0.3) (layer "F.Cu") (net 15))
 (segment (start 50.8 50.8) (end 50.8 55.88) (width 0.5) (layer "F.Cu") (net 7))
 (segment (start 48.895 47.625) (end 50.8 45.72) (width 0.3) (layer "F.Cu") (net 6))
 (segment (start 56.21 80.39) (end 56.21 75.895) (width 0.3) (layer "F.Cu") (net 6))
 (segment (start 56.21 75.895) (end 48.895 68.58) (width 0.3) (layer "F.Cu") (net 6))
 (segment (start 48.895 68.58) (end 48.895 47.625) (width 0.3) (layer "F.Cu") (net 6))
 (segment (start 57.11 81.29) (end 56.21 80.39) (width 0.3) (layer "F.Cu") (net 6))
 (segment (start 71.1 80.04) (end 68.338305 80.04) (width 0.3) (layer "F.Cu") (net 5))
 (segment (start 72.35 81.29) (end 71.1 80.04) (width 0.3) (layer "F.Cu") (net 5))
 (segment (start 68.338305 80.04) (end 57.513305 69.215) (width 0.3) (layer "F.Cu") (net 5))
 (segment (start 57.513305 69.215) (end 57.513305 54.973305) (width 0.3) (layer "F.Cu") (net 5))
 (segment (start 57.513305 54.973305) (end 50.8 48.26) (width 0.3) (layer "F.Cu") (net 5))
 (segment (start 54.2955 86.88) (end 59.82 86.88) (width 0.3) (layer "F.Cu") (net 12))
 (segment (start 52.07 89.1055) (end 54.2955 86.88) (width 0.3) (layer "F.Cu") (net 12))
 (segment (start 51.05 90.1255) (end 52.07 89.1055) (width 0.3) (layer "F.Cu") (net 12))
 (segment (start 51.05 91.6455) (end 51.05 90.1255) (width 0.3) (layer "F.Cu") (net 12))
 (segment (start 54.61 85.5455) (end 51.05 89.1055) (width 0.3) (layer "F.Cu") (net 16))
 (segment (start 54.61 81.29) (end 54.61 85.5455) (width 0.3) (layer "F.Cu") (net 16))
 (segment (start 65.035 92.701366) (end 65.035 93.480634) (width 0.3) (layer "F.Cu") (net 4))
 (segment (start 68.861866 97.3075) (end 73.016714 97.3075) (width 0.3) (layer "F.Cu") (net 4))
 (segment (start 64.77 88.15) (end 65.744999 88.15) (width 0.3) (layer "F.Cu") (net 4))
 (segment (start 72.585 90.42) (end 71.565 91.44) (width 0.3) (layer "F.Cu") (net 4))
 (segment (start 74.175 90.49) (end 72.585 88.9) (width 0.3) (layer "F.Cu") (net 4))
 (segment (start 73.016714 97.3075) (end 74.175 96.149214) (width 0.3) (layer "F.Cu") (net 4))
 (segment (start 65.744999 88.15) (end 67.251365 89.656366) (width 0.3) (layer "F.Cu") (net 4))
 (segment (start 65.035 93.480634) (end 68.861866 97.3075) (width 0.3) (layer "F.Cu") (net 4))
 (segment (start 72.585 88.9) (end 72.585 90.42) (width 0.3) (layer "F.Cu") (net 4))
 (segment (start 67.251365 89.656366) (end 67.251365 90.485001) (width 0.3) (layer "F.Cu") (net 4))
 (segment (start 74.175 96.149214) (end 74.175 90.49) (width 0.3) (layer "F.Cu") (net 4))
 (segment (start 67.251365 90.485001) (end 65.035 92.701366) (width 0.3) (layer "F.Cu") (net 4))
 (segment (start 69.85 87.185) (end 71.565 88.9) (width 0.3) (layer "F.Cu") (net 3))
 (segment (start 69.85 81.29) (end 69.85 87.185) (width 0.3) (layer "F.Cu") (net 3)))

